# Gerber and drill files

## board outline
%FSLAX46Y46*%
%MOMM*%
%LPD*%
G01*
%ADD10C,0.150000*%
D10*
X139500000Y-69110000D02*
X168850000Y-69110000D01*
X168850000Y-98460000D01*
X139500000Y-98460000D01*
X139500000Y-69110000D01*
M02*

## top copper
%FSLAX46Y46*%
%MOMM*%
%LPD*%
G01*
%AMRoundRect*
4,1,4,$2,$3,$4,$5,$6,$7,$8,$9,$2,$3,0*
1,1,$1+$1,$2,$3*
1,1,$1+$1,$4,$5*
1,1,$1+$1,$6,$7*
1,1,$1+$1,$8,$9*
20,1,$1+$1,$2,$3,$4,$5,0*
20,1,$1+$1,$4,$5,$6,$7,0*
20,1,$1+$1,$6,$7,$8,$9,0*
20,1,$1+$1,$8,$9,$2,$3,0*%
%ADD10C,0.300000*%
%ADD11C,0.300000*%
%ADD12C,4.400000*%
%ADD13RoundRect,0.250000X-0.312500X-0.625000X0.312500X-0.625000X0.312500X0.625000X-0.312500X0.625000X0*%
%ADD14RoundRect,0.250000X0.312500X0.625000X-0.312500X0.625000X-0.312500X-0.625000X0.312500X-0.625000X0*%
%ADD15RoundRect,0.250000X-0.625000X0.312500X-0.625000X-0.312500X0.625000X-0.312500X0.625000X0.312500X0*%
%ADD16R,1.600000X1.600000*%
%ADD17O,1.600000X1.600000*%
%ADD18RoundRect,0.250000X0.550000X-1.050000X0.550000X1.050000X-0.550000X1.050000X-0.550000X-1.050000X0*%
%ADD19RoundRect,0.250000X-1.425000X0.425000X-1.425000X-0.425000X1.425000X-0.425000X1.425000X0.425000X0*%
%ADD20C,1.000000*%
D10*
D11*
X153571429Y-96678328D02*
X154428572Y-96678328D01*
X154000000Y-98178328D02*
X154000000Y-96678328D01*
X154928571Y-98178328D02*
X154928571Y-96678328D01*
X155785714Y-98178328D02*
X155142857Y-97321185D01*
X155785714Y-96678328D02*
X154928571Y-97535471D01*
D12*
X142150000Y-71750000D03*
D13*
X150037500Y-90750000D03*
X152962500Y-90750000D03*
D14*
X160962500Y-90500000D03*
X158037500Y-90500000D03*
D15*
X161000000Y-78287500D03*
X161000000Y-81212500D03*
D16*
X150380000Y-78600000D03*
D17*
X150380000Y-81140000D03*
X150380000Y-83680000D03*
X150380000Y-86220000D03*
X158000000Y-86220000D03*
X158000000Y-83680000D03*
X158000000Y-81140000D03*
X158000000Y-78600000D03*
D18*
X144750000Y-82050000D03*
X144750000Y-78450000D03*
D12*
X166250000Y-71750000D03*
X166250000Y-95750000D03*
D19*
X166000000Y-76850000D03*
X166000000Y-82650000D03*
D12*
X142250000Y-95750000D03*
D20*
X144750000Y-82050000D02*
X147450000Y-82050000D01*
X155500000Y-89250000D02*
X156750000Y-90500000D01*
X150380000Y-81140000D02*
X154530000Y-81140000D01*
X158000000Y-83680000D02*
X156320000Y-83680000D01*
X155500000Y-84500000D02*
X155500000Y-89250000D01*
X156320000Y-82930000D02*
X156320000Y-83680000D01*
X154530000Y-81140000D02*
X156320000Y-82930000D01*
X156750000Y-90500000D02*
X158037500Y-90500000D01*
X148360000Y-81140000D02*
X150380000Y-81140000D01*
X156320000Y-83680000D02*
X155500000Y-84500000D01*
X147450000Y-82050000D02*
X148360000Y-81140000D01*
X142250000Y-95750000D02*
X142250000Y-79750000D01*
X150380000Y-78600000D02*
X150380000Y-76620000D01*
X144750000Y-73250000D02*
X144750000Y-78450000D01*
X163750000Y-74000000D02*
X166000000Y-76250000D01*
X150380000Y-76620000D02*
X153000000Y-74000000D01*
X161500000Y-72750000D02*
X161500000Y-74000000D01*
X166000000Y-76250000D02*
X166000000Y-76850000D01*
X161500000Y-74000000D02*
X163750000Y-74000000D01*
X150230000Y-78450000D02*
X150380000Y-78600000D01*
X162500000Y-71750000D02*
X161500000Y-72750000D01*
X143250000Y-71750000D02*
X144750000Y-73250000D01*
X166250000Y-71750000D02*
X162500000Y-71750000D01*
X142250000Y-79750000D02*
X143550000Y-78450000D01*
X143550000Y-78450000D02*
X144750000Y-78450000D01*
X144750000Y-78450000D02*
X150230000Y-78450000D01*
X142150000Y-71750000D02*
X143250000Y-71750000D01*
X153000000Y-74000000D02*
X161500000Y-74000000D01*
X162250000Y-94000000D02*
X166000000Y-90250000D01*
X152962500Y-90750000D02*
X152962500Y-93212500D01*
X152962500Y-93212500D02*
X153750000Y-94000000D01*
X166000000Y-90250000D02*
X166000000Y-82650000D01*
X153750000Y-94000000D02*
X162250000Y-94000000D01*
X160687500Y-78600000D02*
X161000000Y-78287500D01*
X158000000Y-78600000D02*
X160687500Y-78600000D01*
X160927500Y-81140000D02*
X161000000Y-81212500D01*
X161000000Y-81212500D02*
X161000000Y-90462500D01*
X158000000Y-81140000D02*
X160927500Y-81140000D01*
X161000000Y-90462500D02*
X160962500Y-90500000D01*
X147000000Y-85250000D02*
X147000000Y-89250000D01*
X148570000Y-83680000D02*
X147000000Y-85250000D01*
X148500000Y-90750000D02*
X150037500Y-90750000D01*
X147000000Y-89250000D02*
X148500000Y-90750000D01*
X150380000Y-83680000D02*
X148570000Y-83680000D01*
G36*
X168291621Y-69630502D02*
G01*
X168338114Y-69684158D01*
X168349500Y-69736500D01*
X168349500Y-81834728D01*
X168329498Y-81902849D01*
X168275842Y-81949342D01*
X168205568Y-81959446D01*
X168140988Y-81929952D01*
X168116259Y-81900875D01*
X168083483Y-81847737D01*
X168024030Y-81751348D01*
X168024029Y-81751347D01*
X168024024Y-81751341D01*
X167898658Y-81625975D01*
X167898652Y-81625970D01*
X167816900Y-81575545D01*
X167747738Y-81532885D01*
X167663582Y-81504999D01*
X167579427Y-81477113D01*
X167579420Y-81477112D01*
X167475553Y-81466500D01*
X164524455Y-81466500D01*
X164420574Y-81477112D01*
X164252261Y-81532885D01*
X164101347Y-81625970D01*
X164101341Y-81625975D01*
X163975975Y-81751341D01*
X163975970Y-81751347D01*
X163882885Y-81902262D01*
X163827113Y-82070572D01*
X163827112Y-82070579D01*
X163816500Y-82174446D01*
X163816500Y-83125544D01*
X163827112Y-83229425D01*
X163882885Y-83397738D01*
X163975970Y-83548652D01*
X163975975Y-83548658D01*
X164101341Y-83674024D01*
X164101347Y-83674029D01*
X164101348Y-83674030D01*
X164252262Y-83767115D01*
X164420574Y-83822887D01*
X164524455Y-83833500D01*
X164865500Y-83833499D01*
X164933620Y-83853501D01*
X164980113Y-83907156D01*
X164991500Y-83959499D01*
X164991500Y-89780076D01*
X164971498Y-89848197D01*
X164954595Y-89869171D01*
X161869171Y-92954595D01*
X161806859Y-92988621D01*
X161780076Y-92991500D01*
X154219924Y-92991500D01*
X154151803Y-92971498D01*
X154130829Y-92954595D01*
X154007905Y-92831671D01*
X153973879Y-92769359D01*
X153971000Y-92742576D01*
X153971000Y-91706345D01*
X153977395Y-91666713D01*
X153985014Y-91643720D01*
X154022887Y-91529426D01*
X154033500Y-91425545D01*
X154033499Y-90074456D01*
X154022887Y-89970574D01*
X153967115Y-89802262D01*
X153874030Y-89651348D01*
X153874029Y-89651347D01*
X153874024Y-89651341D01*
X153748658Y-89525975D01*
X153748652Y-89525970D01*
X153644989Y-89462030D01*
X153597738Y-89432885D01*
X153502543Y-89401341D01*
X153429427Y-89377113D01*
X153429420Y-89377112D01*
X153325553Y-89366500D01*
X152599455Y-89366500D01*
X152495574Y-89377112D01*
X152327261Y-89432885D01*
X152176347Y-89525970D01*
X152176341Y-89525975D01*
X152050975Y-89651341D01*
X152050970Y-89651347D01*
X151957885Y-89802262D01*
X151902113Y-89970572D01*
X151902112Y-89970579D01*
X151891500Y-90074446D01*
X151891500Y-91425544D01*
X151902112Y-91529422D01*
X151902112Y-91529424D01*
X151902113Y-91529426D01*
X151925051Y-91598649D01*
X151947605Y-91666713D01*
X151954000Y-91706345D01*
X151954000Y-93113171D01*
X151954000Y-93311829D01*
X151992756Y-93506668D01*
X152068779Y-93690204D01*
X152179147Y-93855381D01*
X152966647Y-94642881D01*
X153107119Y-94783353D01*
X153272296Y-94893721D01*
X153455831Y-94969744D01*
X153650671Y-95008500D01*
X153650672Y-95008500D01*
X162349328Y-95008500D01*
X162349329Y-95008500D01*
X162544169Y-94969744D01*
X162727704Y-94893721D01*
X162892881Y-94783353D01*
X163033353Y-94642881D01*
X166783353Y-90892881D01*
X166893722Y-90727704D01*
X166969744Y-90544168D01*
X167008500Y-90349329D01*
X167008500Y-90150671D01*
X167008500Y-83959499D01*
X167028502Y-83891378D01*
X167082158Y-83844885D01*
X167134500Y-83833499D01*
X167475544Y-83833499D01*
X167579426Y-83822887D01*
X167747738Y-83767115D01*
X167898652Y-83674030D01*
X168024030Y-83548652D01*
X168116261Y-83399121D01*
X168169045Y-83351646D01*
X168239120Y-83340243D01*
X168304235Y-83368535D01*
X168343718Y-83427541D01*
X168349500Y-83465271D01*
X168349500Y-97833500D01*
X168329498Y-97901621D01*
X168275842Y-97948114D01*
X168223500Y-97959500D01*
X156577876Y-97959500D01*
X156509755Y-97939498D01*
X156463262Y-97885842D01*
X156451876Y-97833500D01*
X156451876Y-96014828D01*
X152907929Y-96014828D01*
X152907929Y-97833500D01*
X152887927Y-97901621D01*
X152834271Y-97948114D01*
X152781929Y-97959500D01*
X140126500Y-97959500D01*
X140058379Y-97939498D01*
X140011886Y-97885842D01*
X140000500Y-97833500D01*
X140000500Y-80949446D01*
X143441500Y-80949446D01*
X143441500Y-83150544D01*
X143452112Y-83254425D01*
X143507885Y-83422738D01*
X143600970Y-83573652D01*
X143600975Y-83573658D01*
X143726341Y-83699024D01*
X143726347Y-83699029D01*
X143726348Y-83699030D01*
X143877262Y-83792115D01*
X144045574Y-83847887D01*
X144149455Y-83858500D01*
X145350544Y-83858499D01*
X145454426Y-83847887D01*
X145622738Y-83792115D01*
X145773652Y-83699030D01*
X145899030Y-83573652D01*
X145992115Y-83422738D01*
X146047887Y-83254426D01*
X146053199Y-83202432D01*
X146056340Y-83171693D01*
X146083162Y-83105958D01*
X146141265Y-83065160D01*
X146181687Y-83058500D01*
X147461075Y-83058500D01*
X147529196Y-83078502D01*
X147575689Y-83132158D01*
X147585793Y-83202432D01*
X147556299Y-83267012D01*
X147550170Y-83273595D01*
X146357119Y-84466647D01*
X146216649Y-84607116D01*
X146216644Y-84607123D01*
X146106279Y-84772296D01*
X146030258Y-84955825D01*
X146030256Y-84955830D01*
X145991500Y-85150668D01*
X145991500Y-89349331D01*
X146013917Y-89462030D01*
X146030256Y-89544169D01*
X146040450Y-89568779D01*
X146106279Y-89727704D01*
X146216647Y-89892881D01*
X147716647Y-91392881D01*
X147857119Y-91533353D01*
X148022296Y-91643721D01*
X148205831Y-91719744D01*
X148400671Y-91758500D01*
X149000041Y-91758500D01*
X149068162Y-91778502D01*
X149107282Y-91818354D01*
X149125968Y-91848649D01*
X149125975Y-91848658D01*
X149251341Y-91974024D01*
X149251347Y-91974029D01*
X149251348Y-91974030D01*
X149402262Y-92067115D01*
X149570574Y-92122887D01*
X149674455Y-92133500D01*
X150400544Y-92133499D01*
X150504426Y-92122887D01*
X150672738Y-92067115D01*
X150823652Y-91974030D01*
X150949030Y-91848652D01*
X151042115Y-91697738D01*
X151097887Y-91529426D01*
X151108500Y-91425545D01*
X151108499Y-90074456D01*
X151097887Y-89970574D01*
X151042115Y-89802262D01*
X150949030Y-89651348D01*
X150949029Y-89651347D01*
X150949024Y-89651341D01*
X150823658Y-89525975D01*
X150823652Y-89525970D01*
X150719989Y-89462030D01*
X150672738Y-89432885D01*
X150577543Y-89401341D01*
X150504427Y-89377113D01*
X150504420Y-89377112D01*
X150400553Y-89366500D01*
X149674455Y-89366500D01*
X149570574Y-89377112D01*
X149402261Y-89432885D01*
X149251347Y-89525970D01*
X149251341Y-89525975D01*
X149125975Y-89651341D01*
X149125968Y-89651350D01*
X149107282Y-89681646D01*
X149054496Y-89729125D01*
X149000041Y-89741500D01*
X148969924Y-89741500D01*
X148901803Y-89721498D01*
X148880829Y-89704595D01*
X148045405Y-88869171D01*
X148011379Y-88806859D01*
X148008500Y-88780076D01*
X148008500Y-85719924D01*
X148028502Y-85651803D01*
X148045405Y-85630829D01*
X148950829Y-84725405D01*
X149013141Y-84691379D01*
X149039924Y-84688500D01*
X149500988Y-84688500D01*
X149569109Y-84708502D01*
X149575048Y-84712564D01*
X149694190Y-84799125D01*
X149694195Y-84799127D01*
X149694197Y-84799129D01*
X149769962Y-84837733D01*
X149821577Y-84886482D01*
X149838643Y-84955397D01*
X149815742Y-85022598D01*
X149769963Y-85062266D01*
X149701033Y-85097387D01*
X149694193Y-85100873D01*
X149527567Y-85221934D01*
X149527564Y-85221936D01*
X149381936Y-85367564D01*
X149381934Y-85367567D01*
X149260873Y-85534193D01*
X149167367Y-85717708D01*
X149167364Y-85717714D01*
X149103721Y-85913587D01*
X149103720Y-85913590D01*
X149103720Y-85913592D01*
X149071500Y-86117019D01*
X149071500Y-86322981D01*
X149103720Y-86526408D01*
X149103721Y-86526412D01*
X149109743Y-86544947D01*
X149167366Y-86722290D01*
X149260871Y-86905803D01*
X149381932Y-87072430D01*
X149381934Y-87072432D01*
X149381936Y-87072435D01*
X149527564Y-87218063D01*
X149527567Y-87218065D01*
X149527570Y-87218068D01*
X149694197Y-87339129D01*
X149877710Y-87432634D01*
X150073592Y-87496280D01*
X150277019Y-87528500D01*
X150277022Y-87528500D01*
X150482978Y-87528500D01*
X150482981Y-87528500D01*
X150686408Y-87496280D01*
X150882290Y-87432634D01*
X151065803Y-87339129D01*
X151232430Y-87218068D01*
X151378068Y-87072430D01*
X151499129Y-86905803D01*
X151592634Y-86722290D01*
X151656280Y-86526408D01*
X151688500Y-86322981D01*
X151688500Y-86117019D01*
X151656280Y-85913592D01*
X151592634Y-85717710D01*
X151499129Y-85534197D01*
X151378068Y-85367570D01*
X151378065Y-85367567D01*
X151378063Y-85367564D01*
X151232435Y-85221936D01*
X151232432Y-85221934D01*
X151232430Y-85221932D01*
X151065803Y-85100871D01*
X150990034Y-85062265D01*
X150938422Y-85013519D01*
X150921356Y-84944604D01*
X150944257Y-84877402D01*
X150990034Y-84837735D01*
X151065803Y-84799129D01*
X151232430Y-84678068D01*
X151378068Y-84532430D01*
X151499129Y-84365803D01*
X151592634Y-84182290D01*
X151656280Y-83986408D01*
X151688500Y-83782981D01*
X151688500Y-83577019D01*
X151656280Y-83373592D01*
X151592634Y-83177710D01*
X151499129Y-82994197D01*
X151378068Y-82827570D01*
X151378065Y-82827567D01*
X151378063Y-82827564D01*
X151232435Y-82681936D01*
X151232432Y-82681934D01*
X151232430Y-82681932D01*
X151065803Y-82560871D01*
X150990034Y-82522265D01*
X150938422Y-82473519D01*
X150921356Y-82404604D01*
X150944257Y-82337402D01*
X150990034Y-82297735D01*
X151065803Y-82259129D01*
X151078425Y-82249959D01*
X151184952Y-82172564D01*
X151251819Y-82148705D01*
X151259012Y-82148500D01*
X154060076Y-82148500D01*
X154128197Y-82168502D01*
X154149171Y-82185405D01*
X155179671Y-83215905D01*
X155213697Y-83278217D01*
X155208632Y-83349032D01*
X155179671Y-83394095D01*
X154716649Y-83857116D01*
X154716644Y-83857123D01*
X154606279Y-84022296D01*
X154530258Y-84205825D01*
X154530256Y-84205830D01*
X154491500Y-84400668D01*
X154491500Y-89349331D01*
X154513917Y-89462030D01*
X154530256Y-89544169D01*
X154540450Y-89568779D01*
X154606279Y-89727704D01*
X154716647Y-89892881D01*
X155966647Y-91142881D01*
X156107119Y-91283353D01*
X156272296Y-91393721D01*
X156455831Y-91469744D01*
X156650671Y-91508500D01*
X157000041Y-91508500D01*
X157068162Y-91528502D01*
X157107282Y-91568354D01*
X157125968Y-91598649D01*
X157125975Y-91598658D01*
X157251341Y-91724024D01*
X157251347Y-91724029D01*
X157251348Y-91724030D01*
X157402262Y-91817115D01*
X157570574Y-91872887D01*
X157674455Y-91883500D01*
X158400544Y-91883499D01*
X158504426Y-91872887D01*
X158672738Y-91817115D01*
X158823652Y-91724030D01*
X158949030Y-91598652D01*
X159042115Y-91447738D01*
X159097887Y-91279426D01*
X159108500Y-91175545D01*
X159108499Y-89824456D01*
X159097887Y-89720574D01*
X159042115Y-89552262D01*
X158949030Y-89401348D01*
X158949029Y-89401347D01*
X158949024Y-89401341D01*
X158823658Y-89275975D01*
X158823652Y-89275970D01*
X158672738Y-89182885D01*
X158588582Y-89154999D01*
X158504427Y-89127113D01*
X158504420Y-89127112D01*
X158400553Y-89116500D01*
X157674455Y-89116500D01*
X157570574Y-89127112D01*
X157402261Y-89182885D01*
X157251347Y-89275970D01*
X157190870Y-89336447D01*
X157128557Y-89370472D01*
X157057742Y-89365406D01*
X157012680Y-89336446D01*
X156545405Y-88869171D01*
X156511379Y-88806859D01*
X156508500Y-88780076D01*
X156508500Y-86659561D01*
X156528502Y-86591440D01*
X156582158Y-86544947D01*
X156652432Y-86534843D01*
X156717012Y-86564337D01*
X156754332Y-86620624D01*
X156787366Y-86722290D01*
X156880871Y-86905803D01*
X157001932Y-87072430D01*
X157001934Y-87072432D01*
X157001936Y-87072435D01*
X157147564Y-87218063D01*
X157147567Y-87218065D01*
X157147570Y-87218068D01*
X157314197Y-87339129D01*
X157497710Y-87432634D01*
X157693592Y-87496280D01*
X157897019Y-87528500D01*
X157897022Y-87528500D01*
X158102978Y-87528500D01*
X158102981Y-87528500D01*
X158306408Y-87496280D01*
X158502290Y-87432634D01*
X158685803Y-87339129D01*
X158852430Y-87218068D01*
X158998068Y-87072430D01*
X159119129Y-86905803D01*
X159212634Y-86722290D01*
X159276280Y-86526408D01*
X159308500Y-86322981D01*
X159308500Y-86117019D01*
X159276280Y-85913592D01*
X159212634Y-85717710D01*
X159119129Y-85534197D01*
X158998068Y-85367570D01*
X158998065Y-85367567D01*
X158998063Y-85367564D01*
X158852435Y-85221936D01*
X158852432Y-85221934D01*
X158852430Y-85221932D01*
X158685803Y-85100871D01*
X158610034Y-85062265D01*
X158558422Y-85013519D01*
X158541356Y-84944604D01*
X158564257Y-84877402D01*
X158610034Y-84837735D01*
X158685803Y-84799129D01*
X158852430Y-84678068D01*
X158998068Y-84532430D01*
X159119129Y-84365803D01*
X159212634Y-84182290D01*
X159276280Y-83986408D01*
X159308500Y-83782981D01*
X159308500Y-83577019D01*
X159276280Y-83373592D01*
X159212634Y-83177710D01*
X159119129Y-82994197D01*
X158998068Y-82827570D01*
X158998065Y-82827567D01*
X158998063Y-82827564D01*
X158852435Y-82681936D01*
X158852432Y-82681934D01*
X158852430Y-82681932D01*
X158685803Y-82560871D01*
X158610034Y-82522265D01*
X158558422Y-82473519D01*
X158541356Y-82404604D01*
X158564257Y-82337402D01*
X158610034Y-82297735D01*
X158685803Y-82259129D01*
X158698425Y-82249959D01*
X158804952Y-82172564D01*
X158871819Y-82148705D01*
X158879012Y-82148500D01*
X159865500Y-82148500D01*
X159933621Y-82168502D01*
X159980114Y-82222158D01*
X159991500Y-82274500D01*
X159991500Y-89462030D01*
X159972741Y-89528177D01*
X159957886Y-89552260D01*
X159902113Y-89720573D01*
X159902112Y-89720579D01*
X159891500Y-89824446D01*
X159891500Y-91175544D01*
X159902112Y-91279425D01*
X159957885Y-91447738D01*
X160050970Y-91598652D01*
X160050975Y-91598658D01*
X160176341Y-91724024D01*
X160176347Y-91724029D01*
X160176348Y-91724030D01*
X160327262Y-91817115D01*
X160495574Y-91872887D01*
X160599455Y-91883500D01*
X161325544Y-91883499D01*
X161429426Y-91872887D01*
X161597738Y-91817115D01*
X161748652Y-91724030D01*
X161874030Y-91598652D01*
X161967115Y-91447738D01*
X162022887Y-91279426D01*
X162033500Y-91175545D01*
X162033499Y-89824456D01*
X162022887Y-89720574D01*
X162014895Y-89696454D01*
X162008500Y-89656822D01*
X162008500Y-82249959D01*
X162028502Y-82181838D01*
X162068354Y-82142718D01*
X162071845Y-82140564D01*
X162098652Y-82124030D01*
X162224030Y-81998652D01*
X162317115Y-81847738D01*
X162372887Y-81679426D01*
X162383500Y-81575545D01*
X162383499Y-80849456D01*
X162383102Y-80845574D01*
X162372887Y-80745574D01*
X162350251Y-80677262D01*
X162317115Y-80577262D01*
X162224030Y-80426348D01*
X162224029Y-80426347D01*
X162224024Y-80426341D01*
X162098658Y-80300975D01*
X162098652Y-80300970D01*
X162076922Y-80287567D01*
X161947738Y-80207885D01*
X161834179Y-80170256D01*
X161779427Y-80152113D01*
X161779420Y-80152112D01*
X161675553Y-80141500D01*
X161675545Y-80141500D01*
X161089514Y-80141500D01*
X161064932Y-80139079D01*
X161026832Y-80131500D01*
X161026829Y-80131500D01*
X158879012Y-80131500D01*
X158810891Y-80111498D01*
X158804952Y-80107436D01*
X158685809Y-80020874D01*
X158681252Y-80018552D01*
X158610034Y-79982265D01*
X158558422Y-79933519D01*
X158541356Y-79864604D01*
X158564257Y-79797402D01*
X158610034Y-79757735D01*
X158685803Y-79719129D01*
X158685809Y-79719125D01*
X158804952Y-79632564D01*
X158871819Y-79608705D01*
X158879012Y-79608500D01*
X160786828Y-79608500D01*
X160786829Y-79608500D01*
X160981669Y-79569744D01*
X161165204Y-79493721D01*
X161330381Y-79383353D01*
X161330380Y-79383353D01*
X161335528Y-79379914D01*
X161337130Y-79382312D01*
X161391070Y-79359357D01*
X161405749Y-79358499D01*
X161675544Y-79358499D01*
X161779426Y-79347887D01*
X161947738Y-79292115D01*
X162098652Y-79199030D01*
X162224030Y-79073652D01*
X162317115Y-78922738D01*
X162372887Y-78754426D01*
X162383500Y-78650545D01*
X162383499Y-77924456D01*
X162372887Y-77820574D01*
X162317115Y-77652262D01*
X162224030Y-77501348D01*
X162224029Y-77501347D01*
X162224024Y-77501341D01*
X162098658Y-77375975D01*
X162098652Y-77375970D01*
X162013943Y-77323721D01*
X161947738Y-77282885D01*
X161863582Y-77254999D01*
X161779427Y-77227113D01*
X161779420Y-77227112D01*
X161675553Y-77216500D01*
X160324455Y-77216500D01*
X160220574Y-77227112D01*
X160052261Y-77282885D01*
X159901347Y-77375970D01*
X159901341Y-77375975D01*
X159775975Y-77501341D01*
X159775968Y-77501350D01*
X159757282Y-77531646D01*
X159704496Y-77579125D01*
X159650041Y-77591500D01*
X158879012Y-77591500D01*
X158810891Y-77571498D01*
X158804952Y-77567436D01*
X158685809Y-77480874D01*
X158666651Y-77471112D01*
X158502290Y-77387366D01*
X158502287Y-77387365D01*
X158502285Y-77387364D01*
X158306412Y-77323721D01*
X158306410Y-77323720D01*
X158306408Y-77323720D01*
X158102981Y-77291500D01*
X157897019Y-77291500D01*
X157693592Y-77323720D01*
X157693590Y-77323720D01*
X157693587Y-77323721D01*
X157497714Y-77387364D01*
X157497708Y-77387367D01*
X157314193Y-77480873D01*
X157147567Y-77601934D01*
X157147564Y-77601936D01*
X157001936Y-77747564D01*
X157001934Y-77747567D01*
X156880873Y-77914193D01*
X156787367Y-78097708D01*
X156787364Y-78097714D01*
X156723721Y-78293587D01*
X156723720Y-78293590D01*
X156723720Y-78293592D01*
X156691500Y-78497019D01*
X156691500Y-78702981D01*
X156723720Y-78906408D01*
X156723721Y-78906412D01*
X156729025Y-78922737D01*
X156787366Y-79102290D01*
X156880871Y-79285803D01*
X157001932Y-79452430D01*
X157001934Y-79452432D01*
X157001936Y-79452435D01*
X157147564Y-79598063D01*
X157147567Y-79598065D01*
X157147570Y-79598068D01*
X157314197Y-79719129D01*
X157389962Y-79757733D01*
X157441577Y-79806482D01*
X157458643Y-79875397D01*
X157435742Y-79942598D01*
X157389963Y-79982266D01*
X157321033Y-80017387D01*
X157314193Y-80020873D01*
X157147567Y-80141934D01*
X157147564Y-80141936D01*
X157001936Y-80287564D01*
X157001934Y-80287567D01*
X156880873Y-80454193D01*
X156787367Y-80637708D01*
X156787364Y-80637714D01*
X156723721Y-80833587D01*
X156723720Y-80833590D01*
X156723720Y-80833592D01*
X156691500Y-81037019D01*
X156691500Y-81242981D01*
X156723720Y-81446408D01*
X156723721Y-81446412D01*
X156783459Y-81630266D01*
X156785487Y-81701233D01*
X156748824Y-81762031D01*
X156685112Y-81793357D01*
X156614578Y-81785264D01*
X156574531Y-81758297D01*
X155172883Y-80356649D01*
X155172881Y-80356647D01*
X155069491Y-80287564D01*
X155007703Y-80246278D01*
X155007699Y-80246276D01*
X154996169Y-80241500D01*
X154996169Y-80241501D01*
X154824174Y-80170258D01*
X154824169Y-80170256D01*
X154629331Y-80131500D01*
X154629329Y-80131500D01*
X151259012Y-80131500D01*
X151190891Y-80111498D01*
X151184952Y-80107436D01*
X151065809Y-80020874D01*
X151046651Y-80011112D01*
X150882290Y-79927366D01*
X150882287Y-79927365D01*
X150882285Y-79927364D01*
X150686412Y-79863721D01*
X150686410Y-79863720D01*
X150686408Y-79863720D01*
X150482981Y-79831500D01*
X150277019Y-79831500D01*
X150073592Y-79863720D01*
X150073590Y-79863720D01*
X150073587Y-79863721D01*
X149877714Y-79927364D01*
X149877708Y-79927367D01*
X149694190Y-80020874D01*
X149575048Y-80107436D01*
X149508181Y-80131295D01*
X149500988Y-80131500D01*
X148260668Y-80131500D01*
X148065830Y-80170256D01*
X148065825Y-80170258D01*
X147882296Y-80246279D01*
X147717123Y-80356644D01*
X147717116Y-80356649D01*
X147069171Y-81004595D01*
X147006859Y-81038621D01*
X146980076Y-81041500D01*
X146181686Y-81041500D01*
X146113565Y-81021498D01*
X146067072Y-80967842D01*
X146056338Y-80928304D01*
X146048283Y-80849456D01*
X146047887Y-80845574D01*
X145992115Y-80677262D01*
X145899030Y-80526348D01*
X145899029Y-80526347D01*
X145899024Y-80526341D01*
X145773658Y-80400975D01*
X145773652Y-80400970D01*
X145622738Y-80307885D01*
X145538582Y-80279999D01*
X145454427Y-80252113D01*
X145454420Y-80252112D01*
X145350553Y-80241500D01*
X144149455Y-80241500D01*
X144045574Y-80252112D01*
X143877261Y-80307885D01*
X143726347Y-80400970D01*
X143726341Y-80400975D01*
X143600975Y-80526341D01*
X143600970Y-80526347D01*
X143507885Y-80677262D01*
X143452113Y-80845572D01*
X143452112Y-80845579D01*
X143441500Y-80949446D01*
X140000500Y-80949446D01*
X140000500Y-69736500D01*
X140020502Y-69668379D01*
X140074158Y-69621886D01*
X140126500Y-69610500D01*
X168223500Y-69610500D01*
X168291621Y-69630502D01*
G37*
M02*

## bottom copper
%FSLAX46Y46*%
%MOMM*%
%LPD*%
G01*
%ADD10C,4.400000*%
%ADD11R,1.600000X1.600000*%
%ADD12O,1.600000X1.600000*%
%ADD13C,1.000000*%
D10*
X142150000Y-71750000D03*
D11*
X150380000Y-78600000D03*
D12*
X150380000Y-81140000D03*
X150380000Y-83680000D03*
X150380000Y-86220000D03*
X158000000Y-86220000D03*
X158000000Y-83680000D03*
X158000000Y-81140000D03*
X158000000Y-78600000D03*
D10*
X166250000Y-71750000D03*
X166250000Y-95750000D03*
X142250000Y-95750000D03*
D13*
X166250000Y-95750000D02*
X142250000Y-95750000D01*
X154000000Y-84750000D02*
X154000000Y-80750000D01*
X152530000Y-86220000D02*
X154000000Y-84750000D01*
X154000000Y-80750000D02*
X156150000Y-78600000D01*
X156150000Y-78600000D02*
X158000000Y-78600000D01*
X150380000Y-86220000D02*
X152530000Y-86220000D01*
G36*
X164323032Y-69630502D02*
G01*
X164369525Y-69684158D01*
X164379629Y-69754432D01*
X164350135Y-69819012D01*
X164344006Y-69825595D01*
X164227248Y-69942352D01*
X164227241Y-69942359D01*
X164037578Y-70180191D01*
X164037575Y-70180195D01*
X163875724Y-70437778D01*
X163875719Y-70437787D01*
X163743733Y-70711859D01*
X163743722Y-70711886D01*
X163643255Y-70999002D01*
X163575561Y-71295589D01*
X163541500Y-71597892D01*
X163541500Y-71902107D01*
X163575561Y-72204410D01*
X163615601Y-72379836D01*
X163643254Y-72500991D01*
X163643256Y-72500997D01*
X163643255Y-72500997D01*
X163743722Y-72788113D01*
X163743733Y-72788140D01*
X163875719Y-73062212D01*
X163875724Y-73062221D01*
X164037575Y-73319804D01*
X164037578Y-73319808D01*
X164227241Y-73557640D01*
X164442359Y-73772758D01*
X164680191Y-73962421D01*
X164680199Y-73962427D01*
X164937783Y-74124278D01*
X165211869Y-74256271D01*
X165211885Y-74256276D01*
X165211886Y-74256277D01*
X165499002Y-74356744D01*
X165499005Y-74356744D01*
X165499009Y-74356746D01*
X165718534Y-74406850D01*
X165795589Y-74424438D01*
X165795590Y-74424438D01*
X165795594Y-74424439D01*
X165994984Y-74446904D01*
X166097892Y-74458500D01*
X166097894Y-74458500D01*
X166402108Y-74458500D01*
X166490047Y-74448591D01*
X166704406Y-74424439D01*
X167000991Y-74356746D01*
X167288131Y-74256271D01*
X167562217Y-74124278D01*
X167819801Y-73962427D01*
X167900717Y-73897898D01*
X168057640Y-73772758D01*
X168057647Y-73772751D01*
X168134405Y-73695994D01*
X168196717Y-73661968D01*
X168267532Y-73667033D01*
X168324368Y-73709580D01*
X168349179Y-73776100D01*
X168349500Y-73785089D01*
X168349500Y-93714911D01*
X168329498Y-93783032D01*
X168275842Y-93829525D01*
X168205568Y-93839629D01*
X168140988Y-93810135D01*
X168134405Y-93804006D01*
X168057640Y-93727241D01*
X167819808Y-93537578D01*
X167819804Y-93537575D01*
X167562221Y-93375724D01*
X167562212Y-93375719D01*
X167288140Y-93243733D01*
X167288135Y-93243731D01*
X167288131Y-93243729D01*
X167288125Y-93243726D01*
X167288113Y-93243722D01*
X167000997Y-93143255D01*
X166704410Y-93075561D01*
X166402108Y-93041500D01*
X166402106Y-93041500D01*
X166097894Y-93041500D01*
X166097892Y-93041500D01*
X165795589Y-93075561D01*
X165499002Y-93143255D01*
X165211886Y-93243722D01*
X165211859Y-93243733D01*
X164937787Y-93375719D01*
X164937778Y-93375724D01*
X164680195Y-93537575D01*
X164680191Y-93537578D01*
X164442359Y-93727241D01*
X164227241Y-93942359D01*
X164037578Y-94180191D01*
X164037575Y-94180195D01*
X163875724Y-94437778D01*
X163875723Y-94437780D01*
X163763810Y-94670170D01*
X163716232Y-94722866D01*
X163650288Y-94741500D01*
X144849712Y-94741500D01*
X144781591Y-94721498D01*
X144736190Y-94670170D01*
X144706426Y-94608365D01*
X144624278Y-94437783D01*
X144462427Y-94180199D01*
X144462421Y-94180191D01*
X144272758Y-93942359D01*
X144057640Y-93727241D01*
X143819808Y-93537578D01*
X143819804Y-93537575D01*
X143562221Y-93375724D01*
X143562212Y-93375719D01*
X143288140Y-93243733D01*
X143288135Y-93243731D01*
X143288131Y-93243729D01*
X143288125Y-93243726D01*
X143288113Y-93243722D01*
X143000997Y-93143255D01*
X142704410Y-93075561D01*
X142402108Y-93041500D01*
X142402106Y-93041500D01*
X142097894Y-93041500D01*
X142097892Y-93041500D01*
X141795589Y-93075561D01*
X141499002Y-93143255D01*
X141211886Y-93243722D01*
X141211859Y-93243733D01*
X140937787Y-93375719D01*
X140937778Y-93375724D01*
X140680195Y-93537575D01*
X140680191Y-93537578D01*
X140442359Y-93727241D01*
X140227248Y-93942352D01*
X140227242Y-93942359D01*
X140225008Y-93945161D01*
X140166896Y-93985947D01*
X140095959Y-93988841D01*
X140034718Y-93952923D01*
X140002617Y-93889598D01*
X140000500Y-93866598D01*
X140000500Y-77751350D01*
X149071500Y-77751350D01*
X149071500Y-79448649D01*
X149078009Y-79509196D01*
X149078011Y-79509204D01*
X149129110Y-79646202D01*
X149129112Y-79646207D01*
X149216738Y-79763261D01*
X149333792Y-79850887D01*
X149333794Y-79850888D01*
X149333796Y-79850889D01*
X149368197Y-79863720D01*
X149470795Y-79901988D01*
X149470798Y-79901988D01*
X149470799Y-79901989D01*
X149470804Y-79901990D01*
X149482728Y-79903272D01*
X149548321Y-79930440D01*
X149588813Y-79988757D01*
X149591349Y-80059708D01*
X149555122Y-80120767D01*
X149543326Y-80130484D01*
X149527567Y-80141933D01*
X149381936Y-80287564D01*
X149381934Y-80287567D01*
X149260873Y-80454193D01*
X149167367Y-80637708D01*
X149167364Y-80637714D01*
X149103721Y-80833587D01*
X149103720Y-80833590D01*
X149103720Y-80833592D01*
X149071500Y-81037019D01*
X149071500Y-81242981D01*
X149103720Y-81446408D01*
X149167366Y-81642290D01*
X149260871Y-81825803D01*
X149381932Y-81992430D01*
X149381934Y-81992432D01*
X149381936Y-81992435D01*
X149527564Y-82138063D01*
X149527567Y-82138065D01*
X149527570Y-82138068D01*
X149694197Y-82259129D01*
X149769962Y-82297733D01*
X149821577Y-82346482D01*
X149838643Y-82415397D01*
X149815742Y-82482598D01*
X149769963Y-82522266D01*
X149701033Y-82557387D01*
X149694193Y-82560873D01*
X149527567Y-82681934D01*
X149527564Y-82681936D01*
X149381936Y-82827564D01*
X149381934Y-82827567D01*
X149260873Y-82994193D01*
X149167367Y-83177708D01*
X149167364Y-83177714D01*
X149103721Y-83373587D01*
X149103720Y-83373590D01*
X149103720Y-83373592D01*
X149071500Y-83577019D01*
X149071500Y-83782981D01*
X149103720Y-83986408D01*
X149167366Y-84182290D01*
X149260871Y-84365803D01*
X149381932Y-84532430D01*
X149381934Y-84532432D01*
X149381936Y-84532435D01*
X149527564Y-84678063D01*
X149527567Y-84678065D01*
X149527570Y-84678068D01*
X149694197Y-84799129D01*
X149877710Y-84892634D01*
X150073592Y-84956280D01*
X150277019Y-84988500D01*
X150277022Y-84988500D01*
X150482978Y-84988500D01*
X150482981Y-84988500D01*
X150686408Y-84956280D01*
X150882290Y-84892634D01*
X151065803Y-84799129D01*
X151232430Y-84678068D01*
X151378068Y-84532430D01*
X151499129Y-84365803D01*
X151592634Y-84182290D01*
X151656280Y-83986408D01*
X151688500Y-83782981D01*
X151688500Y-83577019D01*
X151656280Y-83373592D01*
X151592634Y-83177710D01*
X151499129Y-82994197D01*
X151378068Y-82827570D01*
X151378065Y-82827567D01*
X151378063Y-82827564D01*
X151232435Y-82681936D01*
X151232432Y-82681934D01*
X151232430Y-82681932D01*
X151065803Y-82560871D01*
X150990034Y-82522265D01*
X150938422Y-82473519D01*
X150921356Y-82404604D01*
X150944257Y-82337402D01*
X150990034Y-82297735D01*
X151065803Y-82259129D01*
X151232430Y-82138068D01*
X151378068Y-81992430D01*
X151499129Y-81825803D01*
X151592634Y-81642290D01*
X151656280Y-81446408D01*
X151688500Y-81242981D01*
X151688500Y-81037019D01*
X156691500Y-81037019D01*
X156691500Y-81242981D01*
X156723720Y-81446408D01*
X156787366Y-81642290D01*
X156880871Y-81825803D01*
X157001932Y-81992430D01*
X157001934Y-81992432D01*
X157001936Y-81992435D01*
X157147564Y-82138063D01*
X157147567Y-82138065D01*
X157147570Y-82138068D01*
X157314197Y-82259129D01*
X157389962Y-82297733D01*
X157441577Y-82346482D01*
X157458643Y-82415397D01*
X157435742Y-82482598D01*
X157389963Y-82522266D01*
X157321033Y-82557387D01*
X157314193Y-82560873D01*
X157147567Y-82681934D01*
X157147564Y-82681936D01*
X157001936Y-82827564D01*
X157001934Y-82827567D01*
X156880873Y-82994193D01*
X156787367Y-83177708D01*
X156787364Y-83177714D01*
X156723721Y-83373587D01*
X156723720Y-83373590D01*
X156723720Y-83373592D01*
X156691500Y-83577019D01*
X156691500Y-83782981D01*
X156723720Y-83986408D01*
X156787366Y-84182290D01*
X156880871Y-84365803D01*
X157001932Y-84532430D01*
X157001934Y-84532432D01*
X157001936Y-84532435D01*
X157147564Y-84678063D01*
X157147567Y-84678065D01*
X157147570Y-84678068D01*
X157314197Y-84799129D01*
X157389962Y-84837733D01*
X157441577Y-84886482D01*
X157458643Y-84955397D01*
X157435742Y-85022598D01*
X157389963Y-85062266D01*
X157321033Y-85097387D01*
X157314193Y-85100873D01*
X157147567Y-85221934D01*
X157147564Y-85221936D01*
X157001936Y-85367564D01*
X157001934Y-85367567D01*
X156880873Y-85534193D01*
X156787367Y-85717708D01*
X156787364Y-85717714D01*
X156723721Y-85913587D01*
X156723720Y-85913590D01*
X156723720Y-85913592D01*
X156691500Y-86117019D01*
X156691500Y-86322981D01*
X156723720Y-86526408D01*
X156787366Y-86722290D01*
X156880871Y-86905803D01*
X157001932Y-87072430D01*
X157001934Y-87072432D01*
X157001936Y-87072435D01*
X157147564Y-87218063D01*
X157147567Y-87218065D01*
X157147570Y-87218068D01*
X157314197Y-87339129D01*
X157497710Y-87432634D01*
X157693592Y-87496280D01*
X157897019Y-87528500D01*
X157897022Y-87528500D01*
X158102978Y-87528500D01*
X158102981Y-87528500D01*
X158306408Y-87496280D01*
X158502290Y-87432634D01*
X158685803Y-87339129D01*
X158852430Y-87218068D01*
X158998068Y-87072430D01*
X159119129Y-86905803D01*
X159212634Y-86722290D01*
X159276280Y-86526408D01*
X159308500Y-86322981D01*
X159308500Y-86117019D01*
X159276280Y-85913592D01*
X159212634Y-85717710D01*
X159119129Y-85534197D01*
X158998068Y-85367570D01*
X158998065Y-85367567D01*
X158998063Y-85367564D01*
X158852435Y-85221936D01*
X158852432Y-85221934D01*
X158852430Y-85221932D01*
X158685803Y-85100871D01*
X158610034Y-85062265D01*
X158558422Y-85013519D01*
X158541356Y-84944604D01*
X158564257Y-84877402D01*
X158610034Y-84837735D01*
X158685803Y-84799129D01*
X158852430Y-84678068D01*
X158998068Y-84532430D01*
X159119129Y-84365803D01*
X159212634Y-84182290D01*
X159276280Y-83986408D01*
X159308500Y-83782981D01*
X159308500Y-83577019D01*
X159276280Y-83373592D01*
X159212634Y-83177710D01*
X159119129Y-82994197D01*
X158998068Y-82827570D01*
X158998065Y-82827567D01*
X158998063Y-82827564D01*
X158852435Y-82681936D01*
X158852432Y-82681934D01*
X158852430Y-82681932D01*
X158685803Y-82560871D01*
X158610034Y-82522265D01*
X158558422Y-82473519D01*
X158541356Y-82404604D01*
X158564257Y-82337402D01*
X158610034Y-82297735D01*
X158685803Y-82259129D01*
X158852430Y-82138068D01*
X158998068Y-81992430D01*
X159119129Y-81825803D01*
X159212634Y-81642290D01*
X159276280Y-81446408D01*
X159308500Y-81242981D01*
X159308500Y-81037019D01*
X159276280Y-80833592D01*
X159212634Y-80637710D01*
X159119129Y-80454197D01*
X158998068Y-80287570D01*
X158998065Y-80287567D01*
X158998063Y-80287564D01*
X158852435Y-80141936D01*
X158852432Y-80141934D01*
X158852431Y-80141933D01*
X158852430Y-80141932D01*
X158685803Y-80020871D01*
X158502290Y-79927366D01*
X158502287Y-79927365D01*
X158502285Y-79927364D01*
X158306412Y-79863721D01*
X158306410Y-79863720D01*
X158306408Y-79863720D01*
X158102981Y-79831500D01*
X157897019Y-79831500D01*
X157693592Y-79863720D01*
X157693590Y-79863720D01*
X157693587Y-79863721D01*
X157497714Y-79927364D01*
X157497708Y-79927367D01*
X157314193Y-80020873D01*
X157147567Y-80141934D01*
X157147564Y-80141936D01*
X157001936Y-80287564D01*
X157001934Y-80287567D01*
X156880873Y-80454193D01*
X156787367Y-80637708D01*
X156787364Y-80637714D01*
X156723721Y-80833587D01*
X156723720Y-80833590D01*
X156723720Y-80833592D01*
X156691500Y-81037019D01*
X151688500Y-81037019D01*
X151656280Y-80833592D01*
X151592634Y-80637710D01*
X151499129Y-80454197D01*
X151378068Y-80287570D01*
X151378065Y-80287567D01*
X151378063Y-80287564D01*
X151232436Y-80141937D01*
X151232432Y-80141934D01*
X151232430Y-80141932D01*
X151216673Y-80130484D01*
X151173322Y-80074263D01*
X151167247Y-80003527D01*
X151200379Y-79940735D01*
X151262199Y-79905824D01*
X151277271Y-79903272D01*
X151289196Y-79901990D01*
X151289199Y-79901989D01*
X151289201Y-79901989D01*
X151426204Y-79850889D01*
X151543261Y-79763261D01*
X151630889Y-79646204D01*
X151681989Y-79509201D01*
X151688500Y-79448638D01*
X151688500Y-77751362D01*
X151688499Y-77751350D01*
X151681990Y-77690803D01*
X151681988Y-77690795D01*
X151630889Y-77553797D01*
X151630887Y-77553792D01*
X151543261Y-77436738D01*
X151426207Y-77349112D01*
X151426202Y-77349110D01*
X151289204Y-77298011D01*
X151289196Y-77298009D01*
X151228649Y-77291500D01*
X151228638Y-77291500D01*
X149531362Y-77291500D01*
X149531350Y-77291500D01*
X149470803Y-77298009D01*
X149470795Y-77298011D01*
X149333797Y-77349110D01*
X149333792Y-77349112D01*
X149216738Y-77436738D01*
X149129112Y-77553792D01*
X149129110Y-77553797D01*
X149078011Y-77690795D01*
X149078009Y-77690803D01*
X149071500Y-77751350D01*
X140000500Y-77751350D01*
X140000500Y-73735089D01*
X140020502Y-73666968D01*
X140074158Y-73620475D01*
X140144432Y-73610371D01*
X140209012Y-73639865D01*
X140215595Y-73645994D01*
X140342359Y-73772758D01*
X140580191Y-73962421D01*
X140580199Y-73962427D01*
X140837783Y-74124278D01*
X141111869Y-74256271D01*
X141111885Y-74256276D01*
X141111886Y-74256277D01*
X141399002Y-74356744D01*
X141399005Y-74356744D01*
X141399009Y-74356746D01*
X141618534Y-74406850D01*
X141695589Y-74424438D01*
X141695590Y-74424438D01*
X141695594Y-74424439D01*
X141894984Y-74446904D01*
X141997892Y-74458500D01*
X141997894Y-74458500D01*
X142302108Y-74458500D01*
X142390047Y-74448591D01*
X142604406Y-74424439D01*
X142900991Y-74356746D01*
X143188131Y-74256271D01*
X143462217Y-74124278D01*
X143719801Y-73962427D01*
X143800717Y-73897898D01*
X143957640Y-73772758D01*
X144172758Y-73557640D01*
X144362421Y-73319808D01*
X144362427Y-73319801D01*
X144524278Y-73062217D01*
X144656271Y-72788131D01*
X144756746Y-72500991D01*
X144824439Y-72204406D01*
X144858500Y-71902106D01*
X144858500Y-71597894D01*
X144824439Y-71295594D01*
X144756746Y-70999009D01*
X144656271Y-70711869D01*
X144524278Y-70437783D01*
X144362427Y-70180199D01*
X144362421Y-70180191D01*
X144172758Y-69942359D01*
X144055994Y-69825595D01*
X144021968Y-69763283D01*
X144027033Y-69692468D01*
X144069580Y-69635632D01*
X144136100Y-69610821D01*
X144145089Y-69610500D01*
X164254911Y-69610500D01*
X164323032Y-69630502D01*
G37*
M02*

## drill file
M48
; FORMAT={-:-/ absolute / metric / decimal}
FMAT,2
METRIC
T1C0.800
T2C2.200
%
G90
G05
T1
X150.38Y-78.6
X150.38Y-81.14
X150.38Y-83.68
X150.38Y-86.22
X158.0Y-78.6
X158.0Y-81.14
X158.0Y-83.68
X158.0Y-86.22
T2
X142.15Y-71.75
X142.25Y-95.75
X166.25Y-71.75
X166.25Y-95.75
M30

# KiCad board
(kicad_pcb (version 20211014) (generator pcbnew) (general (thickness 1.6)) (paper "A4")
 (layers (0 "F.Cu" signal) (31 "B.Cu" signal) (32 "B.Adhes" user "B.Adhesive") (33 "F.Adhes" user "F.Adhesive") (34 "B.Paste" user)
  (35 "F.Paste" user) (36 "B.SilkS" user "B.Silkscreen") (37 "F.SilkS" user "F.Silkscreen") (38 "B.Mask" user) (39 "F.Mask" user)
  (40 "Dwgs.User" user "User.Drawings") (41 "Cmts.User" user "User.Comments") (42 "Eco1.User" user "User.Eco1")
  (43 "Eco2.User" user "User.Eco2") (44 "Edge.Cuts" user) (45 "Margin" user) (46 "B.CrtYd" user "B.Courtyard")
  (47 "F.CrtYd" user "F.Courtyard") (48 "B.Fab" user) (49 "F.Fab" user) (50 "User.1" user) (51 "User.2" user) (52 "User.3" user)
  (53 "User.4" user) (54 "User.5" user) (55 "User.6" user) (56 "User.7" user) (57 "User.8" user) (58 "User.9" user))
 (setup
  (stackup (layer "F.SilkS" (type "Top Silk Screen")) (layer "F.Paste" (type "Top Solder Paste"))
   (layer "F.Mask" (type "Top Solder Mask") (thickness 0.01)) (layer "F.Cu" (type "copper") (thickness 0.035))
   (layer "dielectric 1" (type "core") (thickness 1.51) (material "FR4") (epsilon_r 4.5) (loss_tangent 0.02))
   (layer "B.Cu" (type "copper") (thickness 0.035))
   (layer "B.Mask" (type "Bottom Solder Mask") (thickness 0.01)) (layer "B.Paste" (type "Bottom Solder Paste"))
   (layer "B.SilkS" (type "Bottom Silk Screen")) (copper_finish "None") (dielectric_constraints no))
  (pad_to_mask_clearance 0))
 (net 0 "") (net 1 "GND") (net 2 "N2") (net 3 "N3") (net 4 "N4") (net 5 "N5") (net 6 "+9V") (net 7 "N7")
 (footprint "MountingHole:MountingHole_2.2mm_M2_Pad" (layer "F.Cu") (at 142.15 71.75)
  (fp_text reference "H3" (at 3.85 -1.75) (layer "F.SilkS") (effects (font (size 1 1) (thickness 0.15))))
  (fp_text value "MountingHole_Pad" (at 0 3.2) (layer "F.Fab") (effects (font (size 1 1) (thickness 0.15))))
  (pad "1" thru_hole circle (at 0 0) (size 4.4 4.4) (drill 2.2) (layers *.Cu *.Mask) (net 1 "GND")))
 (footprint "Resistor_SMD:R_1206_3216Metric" (layer "F.Cu") (at 151.5 90.75)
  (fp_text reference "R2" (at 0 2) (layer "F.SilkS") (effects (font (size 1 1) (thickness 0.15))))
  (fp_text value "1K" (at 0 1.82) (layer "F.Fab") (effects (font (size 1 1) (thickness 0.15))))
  (pad "1" smd roundrect (at -1.4625 0) (size 1.125 1.75) (layers "F.Cu" "F.Paste" "F.Mask") (roundrect_rratio 0.2222222222) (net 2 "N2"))
  (pad "2" smd roundrect (at 1.4625 0) (size 1.125 1.75) (layers "F.Cu" "F.Paste" "F.Mask") (roundrect_rratio 0.2222222222) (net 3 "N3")))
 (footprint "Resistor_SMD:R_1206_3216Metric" (layer "F.Cu") (at 159.5 90.5 180)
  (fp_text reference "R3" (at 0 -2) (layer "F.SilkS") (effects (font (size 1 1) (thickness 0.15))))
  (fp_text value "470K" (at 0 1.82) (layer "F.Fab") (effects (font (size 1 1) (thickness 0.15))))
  (pad "1" smd roundrect (at -1.4625 0 180) (size 1.125 1.75) (layers "F.Cu" "F.Paste" "F.Mask") (roundrect_rratio 0.2222222222)
   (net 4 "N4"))
  (pad "2" smd roundrect (at 1.4625 0 180) (size 1.125 1.75) (layers "F.Cu" "F.Paste" "F.Mask") (roundrect_rratio 0.2222222222) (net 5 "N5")))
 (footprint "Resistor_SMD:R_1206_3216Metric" (layer "F.Cu") (at 161 79.75 -90)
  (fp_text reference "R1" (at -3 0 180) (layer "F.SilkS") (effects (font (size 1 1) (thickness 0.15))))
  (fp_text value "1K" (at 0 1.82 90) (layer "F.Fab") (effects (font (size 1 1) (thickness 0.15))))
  (pad "1" smd roundrect (at -1.4625 0 270) (size 1.125 1.75) (layers "F.Cu" "F.Paste" "F.Mask") (roundrect_rratio 0.2222222222)
   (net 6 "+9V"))
  (pad "2" smd roundrect (at 1.4625 0 270) (size 1.125 1.75) (layers "F.Cu" "F.Paste" "F.Mask") (roundrect_rratio 0.2222222222) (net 4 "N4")))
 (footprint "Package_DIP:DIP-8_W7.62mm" (layer "F.Cu") (at 150.38 78.6)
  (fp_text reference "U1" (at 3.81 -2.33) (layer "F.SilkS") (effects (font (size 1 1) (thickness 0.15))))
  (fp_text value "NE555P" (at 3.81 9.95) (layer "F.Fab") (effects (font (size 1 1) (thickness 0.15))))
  (pad "1" thru_hole rect (at 0 0) (size 1.6 1.6) (drill 0.8) (layers *.Cu *.Mask) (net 1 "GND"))
  (pad "2" thru_hole oval (at 0 2.54) (size 1.6 1.6) (drill 0.8) (layers *.Cu *.Mask) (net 5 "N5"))
  (pad "3" thru_hole oval (at 0 5.08) (size 1.6 1.6) (drill 0.8) (layers *.Cu *.Mask) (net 2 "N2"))
  (pad "4" thru_hole oval (at 0 7.62) (size 1.6 1.6) (drill 0.8) (layers *.Cu *.Mask) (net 6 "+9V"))
  (pad "5" thru_hole oval (at 7.62 7.62) (size 1.6 1.6) (drill 0.8) (layers *.Cu *.Mask) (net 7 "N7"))
  (pad "6" thru_hole oval (at 7.62 5.08) (size 1.6 1.6) (drill 0.8) (layers *.Cu *.Mask) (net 5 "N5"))
  (pad "7" thru_hole oval (at 7.62 2.54) (size 1.6 1.6) (drill 0.8) (layers *.Cu *.Mask) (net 4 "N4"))
  (pad "8" thru_hole oval (at 7.62 0) (size 1.6 1.6) (drill 0.8) (layers *.Cu *.Mask) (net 6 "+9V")))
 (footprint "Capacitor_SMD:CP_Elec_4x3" (layer "F.Cu") (at 144.75 80.25 90)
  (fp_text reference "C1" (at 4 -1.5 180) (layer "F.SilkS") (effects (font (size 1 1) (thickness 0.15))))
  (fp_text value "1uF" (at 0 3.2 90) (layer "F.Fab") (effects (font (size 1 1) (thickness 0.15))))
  (pad "1" smd roundrect (at -1.8 0 90) (size 2.6 1.6) (layers "F.Cu" "F.Paste" "F.Mask") (roundrect_rratio 0.15625) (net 5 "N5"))
  (pad "2" smd roundrect (at 1.8 0 90) (size 2.6 1.6) (layers "F.Cu" "F.Paste" "F.Mask") (roundrect_rratio 0.15625) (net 1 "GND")))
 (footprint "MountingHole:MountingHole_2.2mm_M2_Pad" (layer "F.Cu") (at 166.25 71.75)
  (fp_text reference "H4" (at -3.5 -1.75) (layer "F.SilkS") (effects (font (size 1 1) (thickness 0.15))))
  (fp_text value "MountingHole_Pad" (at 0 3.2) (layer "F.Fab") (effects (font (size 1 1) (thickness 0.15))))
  (pad "1" thru_hole circle (at 0 0) (size 4.4 4.4) (drill 2.2) (layers *.Cu *.Mask) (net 1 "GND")))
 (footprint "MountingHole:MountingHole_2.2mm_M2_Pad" (layer "F.Cu") (at 166.25 95.75)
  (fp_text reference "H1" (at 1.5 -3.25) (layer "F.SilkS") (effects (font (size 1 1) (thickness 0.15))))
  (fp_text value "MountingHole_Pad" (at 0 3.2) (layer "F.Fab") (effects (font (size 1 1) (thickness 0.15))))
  (pad "1" thru_hole circle (at 0 0) (size 4.4 4.4) (drill 2.2) (layers *.Cu *.Mask) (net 1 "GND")))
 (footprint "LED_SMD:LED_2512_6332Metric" (layer "F.Cu") (at 166 79.75 -90)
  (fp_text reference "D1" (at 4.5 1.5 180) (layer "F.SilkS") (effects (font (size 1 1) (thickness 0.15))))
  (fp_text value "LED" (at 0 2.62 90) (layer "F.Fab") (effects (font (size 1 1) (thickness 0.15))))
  (pad "1" smd roundrect (at -2.9 0 270) (size 1.35 3.35) (layers "F.Cu" "F.Paste" "F.Mask") (roundrect_rratio 0.1851851852) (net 1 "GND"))
  (pad "2" smd roundrect (at 2.9 0 270) (size 1.35 3.35) (layers "F.Cu" "F.Paste" "F.Mask") (roundrect_rratio 0.1851851852) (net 3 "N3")))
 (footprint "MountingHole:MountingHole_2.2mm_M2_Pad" (layer "F.Cu") (at 142.25 95.75)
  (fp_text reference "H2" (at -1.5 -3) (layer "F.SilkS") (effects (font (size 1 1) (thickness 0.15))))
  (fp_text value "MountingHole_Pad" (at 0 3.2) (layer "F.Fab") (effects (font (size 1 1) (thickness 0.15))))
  (pad "1" thru_hole circle (at 0 0) (size 4.4 4.4) (drill 2.2) (layers *.Cu *.Mask) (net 1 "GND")))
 (gr_rect (start 139.5 69.11) (end 168.85 98.46) (layer "Edge.Cuts") (width 0.15) (fill none))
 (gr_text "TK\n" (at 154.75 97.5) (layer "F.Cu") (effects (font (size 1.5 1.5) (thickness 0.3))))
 (segment (start 144.75 82.05) (end 147.45 82.05) (width 1) (layer "F.Cu") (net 5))
 (segment (start 155.5 89.25) (end 156.75 90.5) (width 1) (layer "F.Cu") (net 5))
 (segment (start 150.38 81.14) (end 154.53 81.14) (width 1) (layer "F.Cu") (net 5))
 (segment (start 158 83.68) (end 156.32 83.68) (width 1) (layer "F.Cu") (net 5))
 (segment (start 155.5 84.5) (end 155.5 89.25) (width 1) (layer "F.Cu") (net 5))
 (segment (start 156.32 82.93) (end 156.32 83.68) (width 1) (layer "F.Cu") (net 5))
 (segment (start 154.53 81.14) (end 156.32 82.93) (width 1) (layer "F.Cu") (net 5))
 (segment (start 156.75 90.5) (end 158.0375 90.5) (width 1) (layer "F.Cu") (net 5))
 (segment (start 148.36 81.14) (end 150.38 81.14) (width 1) (layer "F.Cu") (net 5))
 (segment (start 156.32 83.68) (end 155.5 84.5) (width 1) (layer "F.Cu") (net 5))
 (segment (start 147.45 82.05) (end 148.36 81.14) (width 1) (layer "F.Cu") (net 5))
 (segment (start 142.25 95.75) (end 142.25 79.75) (width 1) (layer "F.Cu") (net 1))
 (segment (start 150.38 78.6) (end 150.38 76.62) (width 1) (layer "F.Cu") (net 1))
 (segment (start 144.75 73.25) (end 144.75 78.45) (width 1) (layer "F.Cu") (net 1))
 (segment (start 163.75 74) (end 166 76.25) (width 1) (layer "F.Cu") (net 1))
 (segment (start 150.38 76.62) (end 153 74) (width 1) (layer "F.Cu") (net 1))
 (segment (start 161.5 72.75) (end 161.5 74) (width 1) (layer "F.Cu") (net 1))
 (segment (start 166 76.25) (end 166 76.85) (width 1) (layer "F.Cu") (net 1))
 (segment (start 161.5 74) (end 163.75 74) (width 1) (layer "F.Cu") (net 1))
 (segment (start 150.23 78.45) (end 150.38 78.6) (width 1) (layer "F.Cu") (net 1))
 (segment (start 162.5 71.75) (end 161.5 72.75) (width 1) (layer "F.Cu") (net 1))
 (segment (start 143.25 71.75) (end 144.75 73.25) (width 1) (layer "F.Cu") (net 1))
 (segment (start 166.25 71.75) (end 162.5 71.75) (width 1) (layer "F.Cu") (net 1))
 (segment (start 142.25 79.75) (end 143.55 78.45) (width 1) (layer "F.Cu") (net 1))
 (segment (start 143.55 78.45) (end 144.75 78.45) (width 1) (layer "F.Cu") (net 1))
 (segment (start 144.75 78.45) (end 150.23 78.45) (width 1) (layer "F.Cu") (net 1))
 (segment (start 142.15 71.75) (end 143.25 71.75) (width 1) (layer "F.Cu") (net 1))
 (segment (start 153 74) (end 161.5 74) (width 1) (layer "F.Cu") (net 1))
 (segment (start 166.25 95.75) (end 142.25 95.75) (width 1) (layer "B.Cu") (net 1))
 (segment (start 162.25 94) (end 166 90.25) (width 1) (layer "F.Cu") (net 3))
 (segment (start 152.9625 90.75) (end 152.9625 93.2125) (width 1) (layer "F.Cu") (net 3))
 (segment (start 152.9625 93.2125) (end 153.75 94) (width 1) (layer "F.Cu") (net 3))
 (segment (start 166 90.25) (end 166 82.65) (width 1) (layer "F.Cu") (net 3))
 (segment (start 153.75 94) (end 162.25 94) (width 1) (layer "F.Cu") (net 3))
 (segment (start 160.6875 78.6) (end 161 78.2875) (width 1) (layer "F.Cu") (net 6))
 (segment (start 158 78.6) (end 160.6875 78.6) (width 1) (layer "F.Cu") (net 6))
 (segment (start 154 84.75) (end 154 80.75) (width 1) (layer "B.Cu") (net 6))
 (segment (start 152.53 86.22) (end 154 84.75) (width 1) (layer "B.Cu") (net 6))
 (segment (start 154 80.75) (end 156.15 78.6) (width 1) (layer "B.Cu") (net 6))
 (segment (start 156.15 78.6) (end 158 78.6) (width 1) (layer "B.Cu") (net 6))
 (segment (start 150.38 86.22) (end 152.53 86.22) (width 1) (layer "B.Cu") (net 6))
 (segment (start 160.9275 81.14) (end 161 81.2125) (width 1) (layer "F.Cu") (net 4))
 (segment (start 161 81.2125) (end 161 90.4625) (width 1) (layer "F.Cu") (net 4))
 (segment (start 158 81.14) (end 160.9275 81.14) (width 1) (layer "F.Cu") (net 4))
 (segment (start 161 90.4625) (end 160.9625 90.5) (width 1) (layer "F.Cu") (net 4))
 (segment (start 147 85.25) (end 147 89.25) (width 1) (layer "F.Cu") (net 2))
 (segment (start 148.57 83.68) (end 147 85.25) (width 1) (layer "F.Cu") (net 2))
 (segment (start 148.5 90.75) (end 150.0375 90.75) (width 1) (layer "F.Cu") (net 2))
 (segment (start 147 89.25) (end 148.5 90.75) (width 1) (layer "F.Cu") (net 2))
 (segment (start 150.38 83.68) (end 148.57 83.68) (width 1) (layer "F.Cu") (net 2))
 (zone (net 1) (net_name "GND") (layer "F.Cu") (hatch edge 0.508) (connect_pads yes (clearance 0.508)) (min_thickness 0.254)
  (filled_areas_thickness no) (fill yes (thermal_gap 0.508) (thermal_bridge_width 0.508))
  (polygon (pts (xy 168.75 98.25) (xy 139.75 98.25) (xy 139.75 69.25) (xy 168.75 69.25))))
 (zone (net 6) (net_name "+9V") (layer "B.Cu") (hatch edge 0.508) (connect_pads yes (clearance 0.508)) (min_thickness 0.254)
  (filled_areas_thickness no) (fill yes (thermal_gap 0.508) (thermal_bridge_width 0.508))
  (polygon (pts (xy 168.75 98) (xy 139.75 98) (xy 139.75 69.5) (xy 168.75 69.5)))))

